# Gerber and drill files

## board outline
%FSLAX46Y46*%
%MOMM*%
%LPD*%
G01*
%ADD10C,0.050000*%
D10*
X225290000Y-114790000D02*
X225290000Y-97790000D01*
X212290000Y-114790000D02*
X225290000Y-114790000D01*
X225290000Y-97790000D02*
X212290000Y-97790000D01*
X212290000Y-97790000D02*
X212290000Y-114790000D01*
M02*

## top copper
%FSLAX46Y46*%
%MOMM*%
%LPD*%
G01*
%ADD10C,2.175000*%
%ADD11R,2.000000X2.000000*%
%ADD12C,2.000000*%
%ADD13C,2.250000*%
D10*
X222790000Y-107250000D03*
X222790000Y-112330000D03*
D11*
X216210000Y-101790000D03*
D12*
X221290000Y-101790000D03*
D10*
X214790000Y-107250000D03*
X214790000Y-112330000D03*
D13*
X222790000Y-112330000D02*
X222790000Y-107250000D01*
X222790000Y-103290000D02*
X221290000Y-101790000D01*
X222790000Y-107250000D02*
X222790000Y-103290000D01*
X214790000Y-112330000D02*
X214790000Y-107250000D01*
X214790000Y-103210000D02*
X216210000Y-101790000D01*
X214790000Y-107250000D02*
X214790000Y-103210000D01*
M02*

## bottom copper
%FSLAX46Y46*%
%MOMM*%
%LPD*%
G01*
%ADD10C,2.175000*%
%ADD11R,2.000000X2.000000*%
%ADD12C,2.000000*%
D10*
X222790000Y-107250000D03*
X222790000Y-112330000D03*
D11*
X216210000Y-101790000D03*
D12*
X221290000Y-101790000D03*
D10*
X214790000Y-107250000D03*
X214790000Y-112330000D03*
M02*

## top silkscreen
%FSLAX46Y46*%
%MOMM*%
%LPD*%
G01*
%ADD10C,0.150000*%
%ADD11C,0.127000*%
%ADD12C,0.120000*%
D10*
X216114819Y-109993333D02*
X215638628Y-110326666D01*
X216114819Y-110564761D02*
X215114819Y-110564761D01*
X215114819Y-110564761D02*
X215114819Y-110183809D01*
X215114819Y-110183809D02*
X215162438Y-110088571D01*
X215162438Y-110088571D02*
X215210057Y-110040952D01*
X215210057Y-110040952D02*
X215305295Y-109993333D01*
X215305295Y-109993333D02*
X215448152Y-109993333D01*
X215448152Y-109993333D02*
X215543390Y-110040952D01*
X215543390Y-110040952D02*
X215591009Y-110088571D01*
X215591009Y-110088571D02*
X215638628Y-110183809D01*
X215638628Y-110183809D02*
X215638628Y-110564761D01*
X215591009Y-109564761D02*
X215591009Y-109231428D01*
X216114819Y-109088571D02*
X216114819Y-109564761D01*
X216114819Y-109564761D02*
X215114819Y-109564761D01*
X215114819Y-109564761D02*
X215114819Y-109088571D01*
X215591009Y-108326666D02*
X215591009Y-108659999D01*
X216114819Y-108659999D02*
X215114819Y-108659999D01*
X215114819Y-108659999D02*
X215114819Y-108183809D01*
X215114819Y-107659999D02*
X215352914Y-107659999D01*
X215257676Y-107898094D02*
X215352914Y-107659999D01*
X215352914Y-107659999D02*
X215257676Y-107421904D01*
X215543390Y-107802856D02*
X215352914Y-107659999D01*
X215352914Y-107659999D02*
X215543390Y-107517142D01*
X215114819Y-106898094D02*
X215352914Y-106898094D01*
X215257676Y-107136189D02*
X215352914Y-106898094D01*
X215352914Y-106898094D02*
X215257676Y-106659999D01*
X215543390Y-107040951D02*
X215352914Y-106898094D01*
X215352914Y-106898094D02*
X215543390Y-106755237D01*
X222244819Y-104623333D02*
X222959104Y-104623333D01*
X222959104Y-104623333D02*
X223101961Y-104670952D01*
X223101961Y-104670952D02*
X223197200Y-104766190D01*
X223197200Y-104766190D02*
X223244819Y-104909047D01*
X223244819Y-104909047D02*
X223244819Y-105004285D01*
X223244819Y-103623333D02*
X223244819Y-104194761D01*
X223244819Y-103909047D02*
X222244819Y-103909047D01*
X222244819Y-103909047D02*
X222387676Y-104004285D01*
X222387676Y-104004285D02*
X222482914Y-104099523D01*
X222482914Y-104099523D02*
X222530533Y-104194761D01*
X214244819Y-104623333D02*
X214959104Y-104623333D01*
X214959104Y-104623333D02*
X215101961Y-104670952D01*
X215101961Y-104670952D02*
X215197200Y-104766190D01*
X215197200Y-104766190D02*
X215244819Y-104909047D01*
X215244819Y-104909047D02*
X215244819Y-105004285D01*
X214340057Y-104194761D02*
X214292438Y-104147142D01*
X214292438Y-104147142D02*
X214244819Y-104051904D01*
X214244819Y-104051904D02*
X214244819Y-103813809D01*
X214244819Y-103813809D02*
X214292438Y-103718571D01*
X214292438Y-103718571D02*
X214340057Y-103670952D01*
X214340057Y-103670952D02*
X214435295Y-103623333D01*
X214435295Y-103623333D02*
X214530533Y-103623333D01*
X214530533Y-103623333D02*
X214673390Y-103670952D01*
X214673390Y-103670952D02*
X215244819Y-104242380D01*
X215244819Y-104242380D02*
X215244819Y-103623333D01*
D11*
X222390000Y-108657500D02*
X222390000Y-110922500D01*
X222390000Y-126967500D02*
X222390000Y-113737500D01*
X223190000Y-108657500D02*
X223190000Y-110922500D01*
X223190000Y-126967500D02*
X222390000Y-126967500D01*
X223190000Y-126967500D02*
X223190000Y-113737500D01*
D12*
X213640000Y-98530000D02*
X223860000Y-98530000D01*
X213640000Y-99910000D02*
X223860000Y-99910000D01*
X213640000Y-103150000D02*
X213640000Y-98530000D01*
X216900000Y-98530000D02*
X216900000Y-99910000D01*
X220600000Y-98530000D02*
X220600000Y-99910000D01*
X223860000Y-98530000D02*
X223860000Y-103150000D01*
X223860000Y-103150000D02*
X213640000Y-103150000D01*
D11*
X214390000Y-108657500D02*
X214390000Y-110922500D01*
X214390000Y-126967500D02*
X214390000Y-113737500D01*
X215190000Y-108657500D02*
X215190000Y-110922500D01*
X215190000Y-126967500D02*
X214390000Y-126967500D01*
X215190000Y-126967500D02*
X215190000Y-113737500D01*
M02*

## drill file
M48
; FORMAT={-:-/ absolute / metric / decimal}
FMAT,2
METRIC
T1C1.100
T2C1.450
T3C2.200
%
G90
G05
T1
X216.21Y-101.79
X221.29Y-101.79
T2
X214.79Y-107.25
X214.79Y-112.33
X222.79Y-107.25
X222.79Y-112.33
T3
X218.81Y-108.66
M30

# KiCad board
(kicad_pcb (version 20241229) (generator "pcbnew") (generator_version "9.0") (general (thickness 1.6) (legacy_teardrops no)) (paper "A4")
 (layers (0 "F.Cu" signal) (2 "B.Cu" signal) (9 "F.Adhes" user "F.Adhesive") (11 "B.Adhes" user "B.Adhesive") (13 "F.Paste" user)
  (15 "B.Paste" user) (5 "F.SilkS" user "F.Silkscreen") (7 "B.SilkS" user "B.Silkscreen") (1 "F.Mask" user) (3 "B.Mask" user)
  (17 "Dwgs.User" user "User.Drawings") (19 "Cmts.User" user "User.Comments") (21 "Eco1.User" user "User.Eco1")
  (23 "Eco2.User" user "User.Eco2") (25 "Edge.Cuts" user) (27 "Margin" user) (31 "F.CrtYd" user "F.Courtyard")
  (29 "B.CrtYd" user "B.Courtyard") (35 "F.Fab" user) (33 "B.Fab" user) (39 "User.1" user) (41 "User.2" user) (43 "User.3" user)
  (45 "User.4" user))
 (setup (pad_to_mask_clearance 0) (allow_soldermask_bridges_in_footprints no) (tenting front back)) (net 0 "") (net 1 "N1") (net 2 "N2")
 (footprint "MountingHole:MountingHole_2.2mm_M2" (layer "F.Cu") (at 218.81 108.66 90)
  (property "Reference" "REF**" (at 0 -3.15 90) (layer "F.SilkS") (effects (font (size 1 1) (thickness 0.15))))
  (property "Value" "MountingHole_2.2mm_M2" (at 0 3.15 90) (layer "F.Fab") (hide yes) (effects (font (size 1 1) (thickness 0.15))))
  (pad "" np_thru_hole circle (at 0 0 90) (size 2.2 2.2) (drill 2.2) (layers "*.Cu" "*.Mask")))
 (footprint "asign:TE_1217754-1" (layer "F.Cu") (at 222.79 109.79)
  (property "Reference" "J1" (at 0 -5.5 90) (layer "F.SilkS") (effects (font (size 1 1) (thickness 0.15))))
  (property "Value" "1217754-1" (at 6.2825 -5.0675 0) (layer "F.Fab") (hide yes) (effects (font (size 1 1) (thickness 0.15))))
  (fp_line (start -0.4 -1.1325) (end -0.4 1.1325) (stroke (width 0.127) (type solid)) (layer "F.SilkS"))
  (fp_line (start -0.4 17.1775) (end -0.4 3.9475) (stroke (width 0.127) (type solid)) (layer "F.SilkS"))
  (fp_line (start 0.4 -1.1325) (end 0.4 1.1325) (stroke (width 0.127) (type solid)) (layer "F.SilkS"))
  (fp_line (start 0.4 17.1775) (end -0.4 17.1775) (stroke (width 0.127) (type solid)) (layer "F.SilkS"))
  (fp_line (start 0.4 17.1775) (end 0.4 3.9475) (stroke (width 0.127) (type solid)) (layer "F.SilkS"))
  (pad "1_1" thru_hole circle (at 0 -2.54) (size 2.175 2.175) (drill 1.45) (layers "*.Cu" "*.Mask") (remove_unused_layers no) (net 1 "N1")
   (solder_mask_margin 0.102))
  (pad "1_2" thru_hole circle (at 0 2.54) (size 2.175 2.175) (drill 1.45) (layers "*.Cu" "*.Mask") (remove_unused_layers no) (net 1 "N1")
   (solder_mask_margin 0.102)))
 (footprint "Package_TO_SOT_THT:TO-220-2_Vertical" (layer "F.Cu") (at 216.21 101.79)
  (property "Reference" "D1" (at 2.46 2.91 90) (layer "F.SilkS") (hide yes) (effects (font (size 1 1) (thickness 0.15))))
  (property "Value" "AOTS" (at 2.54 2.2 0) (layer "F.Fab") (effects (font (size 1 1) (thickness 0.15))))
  (fp_line (start -2.57 -3.26) (end 7.65 -3.26) (stroke (width 0.12) (type solid)) (layer "F.SilkS"))
  (fp_line (start -2.57 -1.88) (end 7.65 -1.88) (stroke (width 0.12) (type solid)) (layer "F.SilkS"))
  (fp_line (start -2.57 1.36) (end -2.57 -3.26) (stroke (width 0.12) (type solid)) (layer "F.SilkS"))
  (fp_line (start 0.69 -3.26) (end 0.69 -1.88) (stroke (width 0.12) (type solid)) (layer "F.SilkS"))
  (fp_line (start 4.39 -3.26) (end 4.39 -1.88) (stroke (width 0.12) (type solid)) (layer "F.SilkS"))
  (fp_line (start 7.65 -3.26) (end 7.65 1.36) (stroke (width 0.12) (type solid)) (layer "F.SilkS"))
  (fp_line (start 7.65 1.36) (end -2.57 1.36) (stroke (width 0.12) (type solid)) (layer "F.SilkS"))
  (pad "1" thru_hole rect (at 0 0) (size 2 2) (drill 1.1) (layers "*.Cu" "*.Mask") (remove_unused_layers no) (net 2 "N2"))
  (pad "2" thru_hole circle (at 5.08 0) (size 2 2) (drill 1.1) (layers "*.Cu" "*.Mask") (remove_unused_layers no) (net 1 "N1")))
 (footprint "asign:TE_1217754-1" (layer "F.Cu") (at 214.79 109.79)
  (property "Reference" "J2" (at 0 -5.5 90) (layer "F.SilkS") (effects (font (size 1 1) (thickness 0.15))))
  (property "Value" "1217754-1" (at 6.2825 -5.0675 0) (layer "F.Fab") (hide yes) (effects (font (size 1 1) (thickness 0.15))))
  (fp_line (start -0.4 -1.1325) (end -0.4 1.1325) (stroke (width 0.127) (type solid)) (layer "F.SilkS"))
  (fp_line (start -0.4 17.1775) (end -0.4 3.9475) (stroke (width 0.127) (type solid)) (layer "F.SilkS"))
  (fp_line (start 0.4 -1.1325) (end 0.4 1.1325) (stroke (width 0.127) (type solid)) (layer "F.SilkS"))
  (fp_line (start 0.4 17.1775) (end -0.4 17.1775) (stroke (width 0.127) (type solid)) (layer "F.SilkS"))
  (fp_line (start 0.4 17.1775) (end 0.4 3.9475) (stroke (width 0.127) (type solid)) (layer "F.SilkS"))
  (pad "1_1" thru_hole circle (at 0 -2.54) (size 2.175 2.175) (drill 1.45) (layers "*.Cu" "*.Mask") (remove_unused_layers no) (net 2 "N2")
   (solder_mask_margin 0.102))
  (pad "1_2" thru_hole circle (at 0 2.54) (size 2.175 2.175) (drill 1.45) (layers "*.Cu" "*.Mask") (remove_unused_layers no) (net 2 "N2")
   (solder_mask_margin 0.102)))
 (gr_line (start 225.29 114.79) (end 225.29 97.79) (stroke (width 0.05) (type default)) (layer "Edge.Cuts"))
 (gr_line (start 212.29 114.79) (end 225.29 114.79) (stroke (width 0.05) (type default)) (layer "Edge.Cuts"))
 (gr_line (start 225.29 97.79) (end 212.29 97.79) (stroke (width 0.05) (type default)) (layer "Edge.Cuts"))
 (gr_line (start 212.29 97.79) (end 212.29 114.79) (stroke (width 0.05) (type default)) (layer "Edge.Cuts"))
 (segment (start 222.79 112.33) (end 222.79 107.25) (width 2.25) (layer "F.Cu") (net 1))
 (segment (start 222.79 103.29) (end 221.29 101.79) (width 2.25) (layer "F.Cu") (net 1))
 (segment (start 222.79 107.25) (end 222.79 103.29) (width 2.25) (layer "F.Cu") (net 1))
 (segment (start 214.79 112.33) (end 214.79 107.25) (width 2.25) (layer "F.Cu") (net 2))
 (segment (start 214.79 103.21) (end 216.21 101.79) (width 2.25) (layer "F.Cu") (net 2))
 (segment (start 214.79 107.25) (end 214.79 103.21) (width 2.25) (layer "F.Cu") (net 2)))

